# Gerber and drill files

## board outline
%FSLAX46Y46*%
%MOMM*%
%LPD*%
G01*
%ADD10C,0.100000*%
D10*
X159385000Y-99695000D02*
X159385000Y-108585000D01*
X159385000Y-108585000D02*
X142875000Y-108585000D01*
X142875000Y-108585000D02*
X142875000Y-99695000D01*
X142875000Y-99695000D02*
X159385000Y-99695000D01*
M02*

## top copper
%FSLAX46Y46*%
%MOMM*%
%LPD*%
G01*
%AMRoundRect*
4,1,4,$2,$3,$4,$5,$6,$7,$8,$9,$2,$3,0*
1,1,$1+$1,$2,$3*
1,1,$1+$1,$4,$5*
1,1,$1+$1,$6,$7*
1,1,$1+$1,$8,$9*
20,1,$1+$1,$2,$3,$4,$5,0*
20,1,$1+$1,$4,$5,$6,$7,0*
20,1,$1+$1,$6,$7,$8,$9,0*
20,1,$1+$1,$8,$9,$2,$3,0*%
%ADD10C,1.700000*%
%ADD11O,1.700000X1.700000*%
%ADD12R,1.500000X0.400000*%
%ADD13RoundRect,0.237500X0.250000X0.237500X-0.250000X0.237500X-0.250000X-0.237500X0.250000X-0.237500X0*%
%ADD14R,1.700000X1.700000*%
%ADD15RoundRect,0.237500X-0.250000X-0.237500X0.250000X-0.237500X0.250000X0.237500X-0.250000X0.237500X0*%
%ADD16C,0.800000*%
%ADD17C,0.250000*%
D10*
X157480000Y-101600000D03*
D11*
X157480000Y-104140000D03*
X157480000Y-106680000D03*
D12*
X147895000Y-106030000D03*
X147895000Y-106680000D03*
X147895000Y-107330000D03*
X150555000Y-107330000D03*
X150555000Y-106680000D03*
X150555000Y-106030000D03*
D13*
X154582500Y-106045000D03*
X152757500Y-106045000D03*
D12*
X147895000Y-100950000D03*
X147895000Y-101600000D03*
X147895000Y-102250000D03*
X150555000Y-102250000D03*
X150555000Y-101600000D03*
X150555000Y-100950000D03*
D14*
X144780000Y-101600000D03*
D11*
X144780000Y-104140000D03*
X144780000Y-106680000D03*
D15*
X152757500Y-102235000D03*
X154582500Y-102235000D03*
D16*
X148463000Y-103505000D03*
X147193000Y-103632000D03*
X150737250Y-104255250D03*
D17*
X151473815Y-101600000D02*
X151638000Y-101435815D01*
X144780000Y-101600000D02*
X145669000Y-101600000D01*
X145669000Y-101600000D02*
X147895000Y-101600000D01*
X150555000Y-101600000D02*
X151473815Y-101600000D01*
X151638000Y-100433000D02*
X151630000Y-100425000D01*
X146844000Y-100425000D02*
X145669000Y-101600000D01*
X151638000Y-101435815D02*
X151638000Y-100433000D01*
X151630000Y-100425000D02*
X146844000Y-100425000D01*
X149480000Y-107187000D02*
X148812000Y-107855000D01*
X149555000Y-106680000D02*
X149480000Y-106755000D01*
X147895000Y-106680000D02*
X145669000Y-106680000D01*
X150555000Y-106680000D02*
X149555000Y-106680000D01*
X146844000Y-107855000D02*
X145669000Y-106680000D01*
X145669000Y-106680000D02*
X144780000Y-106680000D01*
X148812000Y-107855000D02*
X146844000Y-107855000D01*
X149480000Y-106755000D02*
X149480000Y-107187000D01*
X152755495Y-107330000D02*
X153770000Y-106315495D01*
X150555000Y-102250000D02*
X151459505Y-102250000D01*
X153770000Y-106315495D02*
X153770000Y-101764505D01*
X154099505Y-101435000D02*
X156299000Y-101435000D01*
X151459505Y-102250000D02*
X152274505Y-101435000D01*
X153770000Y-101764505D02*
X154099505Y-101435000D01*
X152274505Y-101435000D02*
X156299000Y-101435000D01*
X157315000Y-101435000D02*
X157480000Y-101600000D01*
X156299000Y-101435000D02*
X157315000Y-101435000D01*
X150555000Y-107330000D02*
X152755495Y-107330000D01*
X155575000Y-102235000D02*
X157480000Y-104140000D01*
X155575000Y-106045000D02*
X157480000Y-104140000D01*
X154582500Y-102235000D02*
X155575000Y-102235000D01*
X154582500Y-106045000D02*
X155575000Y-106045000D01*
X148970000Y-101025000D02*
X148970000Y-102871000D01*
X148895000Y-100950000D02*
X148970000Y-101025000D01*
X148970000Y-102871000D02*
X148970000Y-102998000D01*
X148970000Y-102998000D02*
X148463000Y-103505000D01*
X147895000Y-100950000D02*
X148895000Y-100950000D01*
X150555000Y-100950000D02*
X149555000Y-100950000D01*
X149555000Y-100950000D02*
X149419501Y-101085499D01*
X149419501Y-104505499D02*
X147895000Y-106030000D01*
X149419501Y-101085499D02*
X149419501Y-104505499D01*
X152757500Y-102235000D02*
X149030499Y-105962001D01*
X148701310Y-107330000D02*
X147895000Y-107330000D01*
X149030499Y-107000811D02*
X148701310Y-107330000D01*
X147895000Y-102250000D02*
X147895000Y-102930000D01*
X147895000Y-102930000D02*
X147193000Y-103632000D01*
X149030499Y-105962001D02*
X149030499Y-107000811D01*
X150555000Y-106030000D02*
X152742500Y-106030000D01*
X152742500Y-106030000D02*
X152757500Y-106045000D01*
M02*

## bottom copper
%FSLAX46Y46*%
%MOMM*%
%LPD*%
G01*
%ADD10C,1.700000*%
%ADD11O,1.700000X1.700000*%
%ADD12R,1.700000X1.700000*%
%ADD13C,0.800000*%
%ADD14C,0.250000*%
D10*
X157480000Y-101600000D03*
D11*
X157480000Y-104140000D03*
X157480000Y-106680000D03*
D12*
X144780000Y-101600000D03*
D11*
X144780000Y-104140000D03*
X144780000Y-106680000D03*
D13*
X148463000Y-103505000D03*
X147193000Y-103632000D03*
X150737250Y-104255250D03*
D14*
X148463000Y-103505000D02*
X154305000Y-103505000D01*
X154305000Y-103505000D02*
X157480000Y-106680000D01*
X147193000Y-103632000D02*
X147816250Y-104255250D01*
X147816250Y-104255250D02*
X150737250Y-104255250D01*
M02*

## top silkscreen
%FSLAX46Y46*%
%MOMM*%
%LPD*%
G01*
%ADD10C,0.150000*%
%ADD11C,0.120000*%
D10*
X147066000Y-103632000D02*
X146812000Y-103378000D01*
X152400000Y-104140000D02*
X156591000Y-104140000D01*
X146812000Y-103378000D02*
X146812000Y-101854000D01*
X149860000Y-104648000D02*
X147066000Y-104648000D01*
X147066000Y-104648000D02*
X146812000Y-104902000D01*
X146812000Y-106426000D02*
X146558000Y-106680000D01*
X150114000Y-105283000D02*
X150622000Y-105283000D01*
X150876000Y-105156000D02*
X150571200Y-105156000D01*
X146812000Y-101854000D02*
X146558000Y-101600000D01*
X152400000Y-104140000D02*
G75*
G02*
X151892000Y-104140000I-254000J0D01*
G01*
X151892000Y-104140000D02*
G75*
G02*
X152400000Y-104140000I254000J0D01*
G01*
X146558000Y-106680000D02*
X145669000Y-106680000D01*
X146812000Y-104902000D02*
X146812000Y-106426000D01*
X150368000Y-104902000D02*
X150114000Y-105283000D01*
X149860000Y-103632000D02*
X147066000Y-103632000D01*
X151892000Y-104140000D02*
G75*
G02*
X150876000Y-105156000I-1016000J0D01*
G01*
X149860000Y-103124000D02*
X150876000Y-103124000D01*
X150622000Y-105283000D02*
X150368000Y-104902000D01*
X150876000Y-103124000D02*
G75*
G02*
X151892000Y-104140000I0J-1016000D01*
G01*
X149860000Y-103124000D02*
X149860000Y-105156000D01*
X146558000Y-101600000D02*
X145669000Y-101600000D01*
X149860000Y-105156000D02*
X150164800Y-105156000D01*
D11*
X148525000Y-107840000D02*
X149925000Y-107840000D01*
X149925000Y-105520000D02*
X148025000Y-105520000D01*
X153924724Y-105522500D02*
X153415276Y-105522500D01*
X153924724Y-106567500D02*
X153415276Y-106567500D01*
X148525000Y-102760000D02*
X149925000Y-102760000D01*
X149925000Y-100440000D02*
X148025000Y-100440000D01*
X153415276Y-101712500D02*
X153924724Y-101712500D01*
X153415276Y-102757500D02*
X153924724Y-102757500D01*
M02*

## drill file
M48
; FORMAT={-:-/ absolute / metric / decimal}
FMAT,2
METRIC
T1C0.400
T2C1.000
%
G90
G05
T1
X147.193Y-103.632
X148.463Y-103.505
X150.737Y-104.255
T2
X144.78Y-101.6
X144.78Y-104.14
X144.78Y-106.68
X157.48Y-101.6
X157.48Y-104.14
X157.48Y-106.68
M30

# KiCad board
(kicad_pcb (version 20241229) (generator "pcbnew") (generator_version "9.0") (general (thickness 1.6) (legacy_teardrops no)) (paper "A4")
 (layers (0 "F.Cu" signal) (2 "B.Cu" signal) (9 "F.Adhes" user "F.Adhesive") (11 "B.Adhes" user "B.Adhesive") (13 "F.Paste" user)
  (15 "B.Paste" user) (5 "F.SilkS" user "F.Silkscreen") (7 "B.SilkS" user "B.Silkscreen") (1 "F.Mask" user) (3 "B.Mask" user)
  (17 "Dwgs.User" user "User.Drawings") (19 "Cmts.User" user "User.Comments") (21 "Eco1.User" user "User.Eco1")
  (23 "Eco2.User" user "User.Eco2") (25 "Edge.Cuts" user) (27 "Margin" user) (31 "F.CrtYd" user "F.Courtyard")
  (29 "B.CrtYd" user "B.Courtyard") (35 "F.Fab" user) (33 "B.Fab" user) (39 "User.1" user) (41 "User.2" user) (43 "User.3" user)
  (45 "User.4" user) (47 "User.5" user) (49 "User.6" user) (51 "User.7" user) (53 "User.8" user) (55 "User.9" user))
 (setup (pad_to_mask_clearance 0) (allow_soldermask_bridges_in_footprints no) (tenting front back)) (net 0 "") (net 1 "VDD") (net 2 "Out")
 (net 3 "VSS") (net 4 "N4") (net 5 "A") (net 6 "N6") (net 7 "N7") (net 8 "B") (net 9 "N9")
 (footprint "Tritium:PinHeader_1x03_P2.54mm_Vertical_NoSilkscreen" (layer "F.Cu") (at 157.48 101.6)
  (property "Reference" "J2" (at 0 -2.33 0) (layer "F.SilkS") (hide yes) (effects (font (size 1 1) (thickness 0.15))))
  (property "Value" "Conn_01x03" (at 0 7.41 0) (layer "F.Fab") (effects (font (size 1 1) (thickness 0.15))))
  (pad "1" thru_hole circle (at 0 0) (size 1.7 1.7) (drill 1) (layers "*.Cu" "*.Mask") (remove_unused_layers no) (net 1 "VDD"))
  (pad "2" thru_hole oval (at 0 2.54) (size 1.7 1.7) (drill 1) (layers "*.Cu" "*.Mask") (remove_unused_layers no) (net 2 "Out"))
  (pad "3" thru_hole oval (at 0 5.08) (size 1.7 1.7) (drill 1) (layers "*.Cu" "*.Mask") (remove_unused_layers no) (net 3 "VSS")))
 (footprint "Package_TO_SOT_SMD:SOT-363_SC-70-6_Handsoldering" (layer "F.Cu") (at 149.225 106.68)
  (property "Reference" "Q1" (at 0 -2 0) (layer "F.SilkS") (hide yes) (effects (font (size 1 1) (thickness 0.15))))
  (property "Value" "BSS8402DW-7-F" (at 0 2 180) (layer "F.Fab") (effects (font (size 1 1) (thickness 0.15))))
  (fp_line (start -0.7 1.16) (end 0.7 1.16) (stroke (width 0.12) (type solid)) (layer "F.SilkS"))
  (fp_line (start 0.7 -1.16) (end -1.2 -1.16) (stroke (width 0.12) (type solid)) (layer "F.SilkS"))
  (pad "1" smd rect (at -1.33 -0.65) (size 1.5 0.4) (layers "F.Cu" "F.Mask" "F.Paste") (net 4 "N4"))
  (pad "2" smd rect (at -1.33 0) (size 1.5 0.4) (layers "F.Cu" "F.Mask" "F.Paste") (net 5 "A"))
  (pad "3" smd rect (at -1.33 0.65) (size 1.5 0.4) (layers "F.Cu" "F.Mask" "F.Paste") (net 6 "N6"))
  (pad "4" smd rect (at 1.33 0.65) (size 1.5 0.4) (layers "F.Cu" "F.Mask" "F.Paste") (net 1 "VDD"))
  (pad "5" smd rect (at 1.33 0) (size 1.5 0.4) (layers "F.Cu" "F.Mask" "F.Paste") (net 5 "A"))
  (pad "6" smd rect (at 1.33 -0.65) (size 1.5 0.4) (layers "F.Cu" "F.Mask" "F.Paste") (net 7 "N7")))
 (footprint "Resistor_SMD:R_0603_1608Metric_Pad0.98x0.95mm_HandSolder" (layer "F.Cu") (at 153.67 106.045 180)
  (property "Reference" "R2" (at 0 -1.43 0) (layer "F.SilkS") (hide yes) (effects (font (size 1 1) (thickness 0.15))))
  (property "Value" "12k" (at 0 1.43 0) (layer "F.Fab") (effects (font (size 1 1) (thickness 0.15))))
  (fp_line (start -0.254724 0.5225) (end 0.254724 0.5225) (stroke (width 0.12) (type solid)) (layer "F.SilkS"))
  (fp_line (start -0.254724 -0.5225) (end 0.254724 -0.5225) (stroke (width 0.12) (type solid)) (layer "F.SilkS"))
  (pad "1" smd roundrect (at -0.9125 0 180) (size 0.975 0.95) (layers "F.Cu" "F.Mask" "F.Paste") (roundrect_rratio 0.25) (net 2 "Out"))
  (pad "2" smd roundrect (at 0.9125 0 180) (size 0.975 0.95) (layers "F.Cu" "F.Mask" "F.Paste") (roundrect_rratio 0.25) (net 7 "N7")))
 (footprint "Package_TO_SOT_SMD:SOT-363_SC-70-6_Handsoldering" (layer "F.Cu") (at 149.225 101.6)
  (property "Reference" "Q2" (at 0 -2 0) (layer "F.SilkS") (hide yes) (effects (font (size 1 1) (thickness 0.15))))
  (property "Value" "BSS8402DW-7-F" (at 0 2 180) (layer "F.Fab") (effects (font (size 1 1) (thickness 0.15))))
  (fp_line (start -0.7 1.16) (end 0.7 1.16) (stroke (width 0.12) (type solid)) (layer "F.SilkS"))
  (fp_line (start 0.7 -1.16) (end -1.2 -1.16) (stroke (width 0.12) (type solid)) (layer "F.SilkS"))
  (pad "1" smd rect (at -1.33 -0.65) (size 1.5 0.4) (layers "F.Cu" "F.Mask" "F.Paste") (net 3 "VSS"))
  (pad "2" smd rect (at -1.33 0) (size 1.5 0.4) (layers "F.Cu" "F.Mask" "F.Paste") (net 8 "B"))
  (pad "3" smd rect (at -1.33 0.65) (size 1.5 0.4) (layers "F.Cu" "F.Mask" "F.Paste") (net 6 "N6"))
  (pad "4" smd rect (at 1.33 0.65) (size 1.5 0.4) (layers "F.Cu" "F.Mask" "F.Paste") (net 1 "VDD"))
  (pad "5" smd rect (at 1.33 0) (size 1.5 0.4) (layers "F.Cu" "F.Mask" "F.Paste") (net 8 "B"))
  (pad "6" smd rect (at 1.33 -0.65) (size 1.5 0.4) (layers "F.Cu" "F.Mask" "F.Paste") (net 4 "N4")))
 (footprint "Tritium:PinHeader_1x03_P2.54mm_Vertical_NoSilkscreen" (layer "F.Cu") (at 144.78 101.6)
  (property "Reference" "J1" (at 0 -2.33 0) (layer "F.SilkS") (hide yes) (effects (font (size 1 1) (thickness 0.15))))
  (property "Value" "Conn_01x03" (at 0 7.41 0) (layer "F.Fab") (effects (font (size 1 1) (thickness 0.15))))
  (pad "1" thru_hole rect (at 0 0) (size 1.7 1.7) (drill 1) (layers "*.Cu" "*.Mask") (remove_unused_layers no) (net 8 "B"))
  (pad "2" thru_hole oval (at 0 2.54) (size 1.7 1.7) (drill 1) (layers "*.Cu" "*.Mask") (remove_unused_layers no) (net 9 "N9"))
  (pad "3" thru_hole oval (at 0 5.08) (size 1.7 1.7) (drill 1) (layers "*.Cu" "*.Mask") (remove_unused_layers no) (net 5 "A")))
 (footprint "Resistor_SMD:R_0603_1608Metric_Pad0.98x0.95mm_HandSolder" (layer "F.Cu") (at 153.67 102.235)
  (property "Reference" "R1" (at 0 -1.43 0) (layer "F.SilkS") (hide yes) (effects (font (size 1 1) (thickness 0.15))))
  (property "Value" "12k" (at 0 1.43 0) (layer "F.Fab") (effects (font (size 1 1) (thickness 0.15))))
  (fp_line (start -0.254724 -0.5225) (end 0.254724 -0.5225) (stroke (width 0.12) (type solid)) (layer "F.SilkS"))
  (fp_line (start -0.254724 0.5225) (end 0.254724 0.5225) (stroke (width 0.12) (type solid)) (layer "F.SilkS"))
  (pad "1" smd roundrect (at -0.9125 0) (size 0.975 0.95) (layers "F.Cu" "F.Mask" "F.Paste") (roundrect_rratio 0.25) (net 6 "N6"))
  (pad "2" smd roundrect (at 0.9125 0) (size 0.975 0.95) (layers "F.Cu" "F.Mask" "F.Paste") (roundrect_rratio 0.25) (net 2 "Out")))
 (gr_line (start 147.066 103.632) (end 146.812 103.378) (stroke (width 0.15) (type solid)) (layer "F.SilkS"))
 (gr_line (start 152.4 104.14) (end 156.591 104.14) (stroke (width 0.15) (type solid)) (layer "F.SilkS"))
 (gr_line (start 146.812 103.378) (end 146.812 101.854) (stroke (width 0.15) (type solid)) (layer "F.SilkS"))
 (gr_line (start 149.86 104.648) (end 147.066 104.648) (stroke (width 0.15) (type solid)) (layer "F.SilkS"))
 (gr_line (start 147.066 104.648) (end 146.812 104.902) (stroke (width 0.15) (type solid)) (layer "F.SilkS"))
 (gr_line (start 146.812 106.426) (end 146.558 106.68) (stroke (width 0.15) (type solid)) (layer "F.SilkS"))
 (gr_line (start 150.114 105.283) (end 150.622 105.283) (stroke (width 0.15) (type solid)) (layer "F.SilkS"))
 (gr_line (start 150.876 105.156) (end 150.5712 105.156) (stroke (width 0.15) (type solid)) (layer "F.SilkS"))
 (gr_line (start 146.812 101.854) (end 146.558 101.6) (stroke (width 0.15) (type solid)) (layer "F.SilkS"))
 (gr_circle (center 152.146 104.14) (end 152.4 104.14) (stroke (width 0.15) (type solid)) (fill no) (layer "F.SilkS"))
 (gr_line (start 146.558 106.68) (end 145.669 106.68) (stroke (width 0.15) (type solid)) (layer "F.SilkS"))
 (gr_line (start 146.812 104.902) (end 146.812 106.426) (stroke (width 0.15) (type solid)) (layer "F.SilkS"))
 (gr_line (start 150.368 104.902) (end 150.114 105.283) (stroke (width 0.15) (type solid)) (layer "F.SilkS"))
 (gr_line (start 149.86 103.632) (end 147.066 103.632) (stroke (width 0.15) (type solid)) (layer "F.SilkS"))
 (gr_arc (start 151.892 104.14) (mid 151.59442 104.85842) (end 150.876 105.156) (stroke (width 0.15) (type solid)) (layer "F.SilkS"))
 (gr_line (start 149.86 103.124) (end 150.876 103.124) (stroke (width 0.15) (type solid)) (layer "F.SilkS"))
 (gr_line (start 150.622 105.283) (end 150.368 104.902) (stroke (width 0.15) (type solid)) (layer "F.SilkS"))
 (gr_arc (start 150.876 103.124) (mid 151.59442 103.42158) (end 151.892 104.14) (stroke (width 0.15) (type solid)) (layer "F.SilkS"))
 (gr_line (start 149.86 103.124) (end 149.86 105.156) (stroke (width 0.15) (type solid)) (layer "F.SilkS"))
 (gr_line (start 146.558 101.6) (end 145.669 101.6) (stroke (width 0.15) (type solid)) (layer "F.SilkS"))
 (gr_line (start 149.86 105.156) (end 150.1648 105.156) (stroke (width 0.15) (type solid)) (layer "F.SilkS"))
 (gr_line (start 159.385 99.695) (end 159.385 108.585) (stroke (width 0.1) (type solid)) (layer "Edge.Cuts"))
 (gr_line (start 159.385 108.585) (end 142.875 108.585) (stroke (width 0.1) (type solid)) (layer "Edge.Cuts"))
 (gr_line (start 142.875 108.585) (end 142.875 99.695) (stroke (width 0.1) (type solid)) (layer "Edge.Cuts"))
 (gr_line (start 142.875 99.695) (end 159.385 99.695) (stroke (width 0.1) (type solid)) (layer "Edge.Cuts"))
 (segment (start 151.473815 101.6) (end 151.638 101.435815) (width 0.25) (layer "F.Cu") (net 8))
 (segment (start 144.78 101.6) (end 145.669 101.6) (width 0.25) (layer "F.Cu") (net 8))
 (segment (start 145.669 101.6) (end 147.895 101.6) (width 0.25) (layer "F.Cu") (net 8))
 (segment (start 150.555 101.6) (end 151.473815 101.6) (width 0.25) (layer "F.Cu") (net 8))
 (segment (start 151.638 100.433) (end 151.63 100.425) (width 0.25) (layer "F.Cu") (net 8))
 (segment (start 146.844 100.425) (end 145.669 101.6) (width 0.25) (layer "F.Cu") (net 8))
 (segment (start 151.638 101.435815) (end 151.638 100.433) (width 0.25) (layer "F.Cu") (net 8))
 (segment (start 151.63 100.425) (end 146.844 100.425) (width 0.25) (layer "F.Cu") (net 8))
 (segment (start 149.48 107.187) (end 148.812 107.855) (width 0.25) (layer "F.Cu") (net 5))
 (segment (start 149.555 106.68) (end 149.48 106.755) (width 0.25) (layer "F.Cu") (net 5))
 (segment (start 147.895 106.68) (end 145.669 106.68) (width 0.25) (layer "F.Cu") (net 5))
 (segment (start 150.555 106.68) (end 149.555 106.68) (width 0.25) (layer "F.Cu") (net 5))
 (segment (start 146.844 107.855) (end 145.669 106.68) (width 0.25) (layer "F.Cu") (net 5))
 (segment (start 145.669 106.68) (end 144.78 106.68) (width 0.25) (layer "F.Cu") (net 5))
 (segment (start 148.812 107.855) (end 146.844 107.855) (width 0.25) (layer "F.Cu") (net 5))
 (segment (start 149.48 106.755) (end 149.48 107.187) (width 0.25) (layer "F.Cu") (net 5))
 (segment (start 152.755495 107.33) (end 153.77 106.315495) (width 0.25) (layer "F.Cu") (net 1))
 (segment (start 150.555 102.25) (end 151.459505 102.25) (width 0.25) (layer "F.Cu") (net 1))
 (segment (start 153.77 106.315495) (end 153.77 101.764505) (width 0.25) (layer "F.Cu") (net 1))
 (segment (start 154.099505 101.435) (end 156.299 101.435) (width 0.25) (layer "F.Cu") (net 1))
 (segment (start 151.459505 102.25) (end 152.274505 101.435) (width 0.25) (layer "F.Cu") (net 1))
 (segment (start 153.77 101.764505) (end 154.099505 101.435) (width 0.25) (layer "F.Cu") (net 1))
 (segment (start 152.274505 101.435) (end 156.299 101.435) (width 0.25) (layer "F.Cu") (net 1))
 (segment (start 157.315 101.435) (end 157.48 101.6) (width 0.25) (layer "F.Cu") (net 1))
 (segment (start 156.299 101.435) (end 157.315 101.435) (width 0.25) (layer "F.Cu") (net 1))
 (segment (start 150.555 107.33) (end 152.755495 107.33) (width 0.25) (layer "F.Cu") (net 1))
 (segment (start 155.575 102.235) (end 157.48 104.14) (width 0.25) (layer "F.Cu") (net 2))
 (segment (start 155.575 106.045) (end 157.48 104.14) (width 0.25) (layer "F.Cu") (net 2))
 (segment (start 154.5825 102.235) (end 155.575 102.235) (width 0.25) (layer "F.Cu") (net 2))
 (segment (start 154.5825 106.045) (end 155.575 106.045) (width 0.25) (layer "F.Cu") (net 2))
 (segment (start 148.97 101.025) (end 148.97 102.871) (width 0.25) (layer "F.Cu") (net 3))
 (segment (start 148.895 100.95) (end 148.97 101.025) (width 0.25) (layer "F.Cu") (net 3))
 (segment (start 148.97 102.871) (end 148.97 102.998) (width 0.25) (layer "F.Cu") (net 3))
 (segment (start 148.97 102.998) (end 148.463 103.505) (width 0.25) (layer "F.Cu") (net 3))
 (segment (start 147.895 100.95) (end 148.895 100.95) (width 0.25) (layer "F.Cu") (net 3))
 (via (at 148.463 103.505) (size 0.8) (drill 0.4) (layers "F.Cu" "B.Cu") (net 3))
 (segment (start 148.463 103.505) (end 154.305 103.505) (width 0.25) (layer "B.Cu") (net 3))
 (segment (start 154.305 103.505) (end 157.48 106.68) (width 0.25) (layer "B.Cu") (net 3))
 (segment (start 150.555 100.95) (end 149.555 100.95) (width 0.25) (layer "F.Cu") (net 4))
 (segment (start 149.555 100.95) (end 149.419501 101.085499) (width 0.25) (layer "F.Cu") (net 4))
 (segment (start 149.419501 104.505499) (end 147.895 106.03) (width 0.25) (layer "F.Cu") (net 4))
 (segment (start 149.419501 101.085499) (end 149.419501 104.505499) (width 0.25) (layer "F.Cu") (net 4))
 (segment (start 152.7575 102.235) (end 149.030499 105.962001) (width 0.25) (layer "F.Cu") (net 6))
 (segment (start 148.70131 107.33) (end 147.895 107.33) (width 0.25) (layer "F.Cu") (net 6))
 (segment (start 149.030499 107.000811) (end 148.70131 107.33) (width 0.25) (layer "F.Cu") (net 6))
 (segment (start 147.895 102.25) (end 147.895 102.93) (width 0.25) (layer "F.Cu") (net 6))
 (segment (start 147.895 102.93) (end 147.193 103.632) (width 0.25) (layer "F.Cu") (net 6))
 (segment (start 149.030499 105.962001) (end 149.030499 107.000811) (width 0.25) (layer "F.Cu") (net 6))
 (via (at 147.193 103.632) (size 0.8) (drill 0.4) (layers "F.Cu" "B.Cu") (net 6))
 (via (at 150.73725 104.25525) (size 0.8) (drill 0.4) (layers "F.Cu" "B.Cu") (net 6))
 (segment (start 147.193 103.632) (end 147.81625 104.25525) (width 0.25) (layer "B.Cu") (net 6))
 (segment (start 147.81625 104.25525) (end 150.73725 104.25525) (width 0.25) (layer "B.Cu") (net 6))
 (segment (start 150.555 106.03) (end 152.7425 106.03) (width 0.25) (layer "F.Cu") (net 7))
 (segment (start 152.7425 106.03) (end 152.7575 106.045) (width 0.25) (layer "F.Cu") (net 7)))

